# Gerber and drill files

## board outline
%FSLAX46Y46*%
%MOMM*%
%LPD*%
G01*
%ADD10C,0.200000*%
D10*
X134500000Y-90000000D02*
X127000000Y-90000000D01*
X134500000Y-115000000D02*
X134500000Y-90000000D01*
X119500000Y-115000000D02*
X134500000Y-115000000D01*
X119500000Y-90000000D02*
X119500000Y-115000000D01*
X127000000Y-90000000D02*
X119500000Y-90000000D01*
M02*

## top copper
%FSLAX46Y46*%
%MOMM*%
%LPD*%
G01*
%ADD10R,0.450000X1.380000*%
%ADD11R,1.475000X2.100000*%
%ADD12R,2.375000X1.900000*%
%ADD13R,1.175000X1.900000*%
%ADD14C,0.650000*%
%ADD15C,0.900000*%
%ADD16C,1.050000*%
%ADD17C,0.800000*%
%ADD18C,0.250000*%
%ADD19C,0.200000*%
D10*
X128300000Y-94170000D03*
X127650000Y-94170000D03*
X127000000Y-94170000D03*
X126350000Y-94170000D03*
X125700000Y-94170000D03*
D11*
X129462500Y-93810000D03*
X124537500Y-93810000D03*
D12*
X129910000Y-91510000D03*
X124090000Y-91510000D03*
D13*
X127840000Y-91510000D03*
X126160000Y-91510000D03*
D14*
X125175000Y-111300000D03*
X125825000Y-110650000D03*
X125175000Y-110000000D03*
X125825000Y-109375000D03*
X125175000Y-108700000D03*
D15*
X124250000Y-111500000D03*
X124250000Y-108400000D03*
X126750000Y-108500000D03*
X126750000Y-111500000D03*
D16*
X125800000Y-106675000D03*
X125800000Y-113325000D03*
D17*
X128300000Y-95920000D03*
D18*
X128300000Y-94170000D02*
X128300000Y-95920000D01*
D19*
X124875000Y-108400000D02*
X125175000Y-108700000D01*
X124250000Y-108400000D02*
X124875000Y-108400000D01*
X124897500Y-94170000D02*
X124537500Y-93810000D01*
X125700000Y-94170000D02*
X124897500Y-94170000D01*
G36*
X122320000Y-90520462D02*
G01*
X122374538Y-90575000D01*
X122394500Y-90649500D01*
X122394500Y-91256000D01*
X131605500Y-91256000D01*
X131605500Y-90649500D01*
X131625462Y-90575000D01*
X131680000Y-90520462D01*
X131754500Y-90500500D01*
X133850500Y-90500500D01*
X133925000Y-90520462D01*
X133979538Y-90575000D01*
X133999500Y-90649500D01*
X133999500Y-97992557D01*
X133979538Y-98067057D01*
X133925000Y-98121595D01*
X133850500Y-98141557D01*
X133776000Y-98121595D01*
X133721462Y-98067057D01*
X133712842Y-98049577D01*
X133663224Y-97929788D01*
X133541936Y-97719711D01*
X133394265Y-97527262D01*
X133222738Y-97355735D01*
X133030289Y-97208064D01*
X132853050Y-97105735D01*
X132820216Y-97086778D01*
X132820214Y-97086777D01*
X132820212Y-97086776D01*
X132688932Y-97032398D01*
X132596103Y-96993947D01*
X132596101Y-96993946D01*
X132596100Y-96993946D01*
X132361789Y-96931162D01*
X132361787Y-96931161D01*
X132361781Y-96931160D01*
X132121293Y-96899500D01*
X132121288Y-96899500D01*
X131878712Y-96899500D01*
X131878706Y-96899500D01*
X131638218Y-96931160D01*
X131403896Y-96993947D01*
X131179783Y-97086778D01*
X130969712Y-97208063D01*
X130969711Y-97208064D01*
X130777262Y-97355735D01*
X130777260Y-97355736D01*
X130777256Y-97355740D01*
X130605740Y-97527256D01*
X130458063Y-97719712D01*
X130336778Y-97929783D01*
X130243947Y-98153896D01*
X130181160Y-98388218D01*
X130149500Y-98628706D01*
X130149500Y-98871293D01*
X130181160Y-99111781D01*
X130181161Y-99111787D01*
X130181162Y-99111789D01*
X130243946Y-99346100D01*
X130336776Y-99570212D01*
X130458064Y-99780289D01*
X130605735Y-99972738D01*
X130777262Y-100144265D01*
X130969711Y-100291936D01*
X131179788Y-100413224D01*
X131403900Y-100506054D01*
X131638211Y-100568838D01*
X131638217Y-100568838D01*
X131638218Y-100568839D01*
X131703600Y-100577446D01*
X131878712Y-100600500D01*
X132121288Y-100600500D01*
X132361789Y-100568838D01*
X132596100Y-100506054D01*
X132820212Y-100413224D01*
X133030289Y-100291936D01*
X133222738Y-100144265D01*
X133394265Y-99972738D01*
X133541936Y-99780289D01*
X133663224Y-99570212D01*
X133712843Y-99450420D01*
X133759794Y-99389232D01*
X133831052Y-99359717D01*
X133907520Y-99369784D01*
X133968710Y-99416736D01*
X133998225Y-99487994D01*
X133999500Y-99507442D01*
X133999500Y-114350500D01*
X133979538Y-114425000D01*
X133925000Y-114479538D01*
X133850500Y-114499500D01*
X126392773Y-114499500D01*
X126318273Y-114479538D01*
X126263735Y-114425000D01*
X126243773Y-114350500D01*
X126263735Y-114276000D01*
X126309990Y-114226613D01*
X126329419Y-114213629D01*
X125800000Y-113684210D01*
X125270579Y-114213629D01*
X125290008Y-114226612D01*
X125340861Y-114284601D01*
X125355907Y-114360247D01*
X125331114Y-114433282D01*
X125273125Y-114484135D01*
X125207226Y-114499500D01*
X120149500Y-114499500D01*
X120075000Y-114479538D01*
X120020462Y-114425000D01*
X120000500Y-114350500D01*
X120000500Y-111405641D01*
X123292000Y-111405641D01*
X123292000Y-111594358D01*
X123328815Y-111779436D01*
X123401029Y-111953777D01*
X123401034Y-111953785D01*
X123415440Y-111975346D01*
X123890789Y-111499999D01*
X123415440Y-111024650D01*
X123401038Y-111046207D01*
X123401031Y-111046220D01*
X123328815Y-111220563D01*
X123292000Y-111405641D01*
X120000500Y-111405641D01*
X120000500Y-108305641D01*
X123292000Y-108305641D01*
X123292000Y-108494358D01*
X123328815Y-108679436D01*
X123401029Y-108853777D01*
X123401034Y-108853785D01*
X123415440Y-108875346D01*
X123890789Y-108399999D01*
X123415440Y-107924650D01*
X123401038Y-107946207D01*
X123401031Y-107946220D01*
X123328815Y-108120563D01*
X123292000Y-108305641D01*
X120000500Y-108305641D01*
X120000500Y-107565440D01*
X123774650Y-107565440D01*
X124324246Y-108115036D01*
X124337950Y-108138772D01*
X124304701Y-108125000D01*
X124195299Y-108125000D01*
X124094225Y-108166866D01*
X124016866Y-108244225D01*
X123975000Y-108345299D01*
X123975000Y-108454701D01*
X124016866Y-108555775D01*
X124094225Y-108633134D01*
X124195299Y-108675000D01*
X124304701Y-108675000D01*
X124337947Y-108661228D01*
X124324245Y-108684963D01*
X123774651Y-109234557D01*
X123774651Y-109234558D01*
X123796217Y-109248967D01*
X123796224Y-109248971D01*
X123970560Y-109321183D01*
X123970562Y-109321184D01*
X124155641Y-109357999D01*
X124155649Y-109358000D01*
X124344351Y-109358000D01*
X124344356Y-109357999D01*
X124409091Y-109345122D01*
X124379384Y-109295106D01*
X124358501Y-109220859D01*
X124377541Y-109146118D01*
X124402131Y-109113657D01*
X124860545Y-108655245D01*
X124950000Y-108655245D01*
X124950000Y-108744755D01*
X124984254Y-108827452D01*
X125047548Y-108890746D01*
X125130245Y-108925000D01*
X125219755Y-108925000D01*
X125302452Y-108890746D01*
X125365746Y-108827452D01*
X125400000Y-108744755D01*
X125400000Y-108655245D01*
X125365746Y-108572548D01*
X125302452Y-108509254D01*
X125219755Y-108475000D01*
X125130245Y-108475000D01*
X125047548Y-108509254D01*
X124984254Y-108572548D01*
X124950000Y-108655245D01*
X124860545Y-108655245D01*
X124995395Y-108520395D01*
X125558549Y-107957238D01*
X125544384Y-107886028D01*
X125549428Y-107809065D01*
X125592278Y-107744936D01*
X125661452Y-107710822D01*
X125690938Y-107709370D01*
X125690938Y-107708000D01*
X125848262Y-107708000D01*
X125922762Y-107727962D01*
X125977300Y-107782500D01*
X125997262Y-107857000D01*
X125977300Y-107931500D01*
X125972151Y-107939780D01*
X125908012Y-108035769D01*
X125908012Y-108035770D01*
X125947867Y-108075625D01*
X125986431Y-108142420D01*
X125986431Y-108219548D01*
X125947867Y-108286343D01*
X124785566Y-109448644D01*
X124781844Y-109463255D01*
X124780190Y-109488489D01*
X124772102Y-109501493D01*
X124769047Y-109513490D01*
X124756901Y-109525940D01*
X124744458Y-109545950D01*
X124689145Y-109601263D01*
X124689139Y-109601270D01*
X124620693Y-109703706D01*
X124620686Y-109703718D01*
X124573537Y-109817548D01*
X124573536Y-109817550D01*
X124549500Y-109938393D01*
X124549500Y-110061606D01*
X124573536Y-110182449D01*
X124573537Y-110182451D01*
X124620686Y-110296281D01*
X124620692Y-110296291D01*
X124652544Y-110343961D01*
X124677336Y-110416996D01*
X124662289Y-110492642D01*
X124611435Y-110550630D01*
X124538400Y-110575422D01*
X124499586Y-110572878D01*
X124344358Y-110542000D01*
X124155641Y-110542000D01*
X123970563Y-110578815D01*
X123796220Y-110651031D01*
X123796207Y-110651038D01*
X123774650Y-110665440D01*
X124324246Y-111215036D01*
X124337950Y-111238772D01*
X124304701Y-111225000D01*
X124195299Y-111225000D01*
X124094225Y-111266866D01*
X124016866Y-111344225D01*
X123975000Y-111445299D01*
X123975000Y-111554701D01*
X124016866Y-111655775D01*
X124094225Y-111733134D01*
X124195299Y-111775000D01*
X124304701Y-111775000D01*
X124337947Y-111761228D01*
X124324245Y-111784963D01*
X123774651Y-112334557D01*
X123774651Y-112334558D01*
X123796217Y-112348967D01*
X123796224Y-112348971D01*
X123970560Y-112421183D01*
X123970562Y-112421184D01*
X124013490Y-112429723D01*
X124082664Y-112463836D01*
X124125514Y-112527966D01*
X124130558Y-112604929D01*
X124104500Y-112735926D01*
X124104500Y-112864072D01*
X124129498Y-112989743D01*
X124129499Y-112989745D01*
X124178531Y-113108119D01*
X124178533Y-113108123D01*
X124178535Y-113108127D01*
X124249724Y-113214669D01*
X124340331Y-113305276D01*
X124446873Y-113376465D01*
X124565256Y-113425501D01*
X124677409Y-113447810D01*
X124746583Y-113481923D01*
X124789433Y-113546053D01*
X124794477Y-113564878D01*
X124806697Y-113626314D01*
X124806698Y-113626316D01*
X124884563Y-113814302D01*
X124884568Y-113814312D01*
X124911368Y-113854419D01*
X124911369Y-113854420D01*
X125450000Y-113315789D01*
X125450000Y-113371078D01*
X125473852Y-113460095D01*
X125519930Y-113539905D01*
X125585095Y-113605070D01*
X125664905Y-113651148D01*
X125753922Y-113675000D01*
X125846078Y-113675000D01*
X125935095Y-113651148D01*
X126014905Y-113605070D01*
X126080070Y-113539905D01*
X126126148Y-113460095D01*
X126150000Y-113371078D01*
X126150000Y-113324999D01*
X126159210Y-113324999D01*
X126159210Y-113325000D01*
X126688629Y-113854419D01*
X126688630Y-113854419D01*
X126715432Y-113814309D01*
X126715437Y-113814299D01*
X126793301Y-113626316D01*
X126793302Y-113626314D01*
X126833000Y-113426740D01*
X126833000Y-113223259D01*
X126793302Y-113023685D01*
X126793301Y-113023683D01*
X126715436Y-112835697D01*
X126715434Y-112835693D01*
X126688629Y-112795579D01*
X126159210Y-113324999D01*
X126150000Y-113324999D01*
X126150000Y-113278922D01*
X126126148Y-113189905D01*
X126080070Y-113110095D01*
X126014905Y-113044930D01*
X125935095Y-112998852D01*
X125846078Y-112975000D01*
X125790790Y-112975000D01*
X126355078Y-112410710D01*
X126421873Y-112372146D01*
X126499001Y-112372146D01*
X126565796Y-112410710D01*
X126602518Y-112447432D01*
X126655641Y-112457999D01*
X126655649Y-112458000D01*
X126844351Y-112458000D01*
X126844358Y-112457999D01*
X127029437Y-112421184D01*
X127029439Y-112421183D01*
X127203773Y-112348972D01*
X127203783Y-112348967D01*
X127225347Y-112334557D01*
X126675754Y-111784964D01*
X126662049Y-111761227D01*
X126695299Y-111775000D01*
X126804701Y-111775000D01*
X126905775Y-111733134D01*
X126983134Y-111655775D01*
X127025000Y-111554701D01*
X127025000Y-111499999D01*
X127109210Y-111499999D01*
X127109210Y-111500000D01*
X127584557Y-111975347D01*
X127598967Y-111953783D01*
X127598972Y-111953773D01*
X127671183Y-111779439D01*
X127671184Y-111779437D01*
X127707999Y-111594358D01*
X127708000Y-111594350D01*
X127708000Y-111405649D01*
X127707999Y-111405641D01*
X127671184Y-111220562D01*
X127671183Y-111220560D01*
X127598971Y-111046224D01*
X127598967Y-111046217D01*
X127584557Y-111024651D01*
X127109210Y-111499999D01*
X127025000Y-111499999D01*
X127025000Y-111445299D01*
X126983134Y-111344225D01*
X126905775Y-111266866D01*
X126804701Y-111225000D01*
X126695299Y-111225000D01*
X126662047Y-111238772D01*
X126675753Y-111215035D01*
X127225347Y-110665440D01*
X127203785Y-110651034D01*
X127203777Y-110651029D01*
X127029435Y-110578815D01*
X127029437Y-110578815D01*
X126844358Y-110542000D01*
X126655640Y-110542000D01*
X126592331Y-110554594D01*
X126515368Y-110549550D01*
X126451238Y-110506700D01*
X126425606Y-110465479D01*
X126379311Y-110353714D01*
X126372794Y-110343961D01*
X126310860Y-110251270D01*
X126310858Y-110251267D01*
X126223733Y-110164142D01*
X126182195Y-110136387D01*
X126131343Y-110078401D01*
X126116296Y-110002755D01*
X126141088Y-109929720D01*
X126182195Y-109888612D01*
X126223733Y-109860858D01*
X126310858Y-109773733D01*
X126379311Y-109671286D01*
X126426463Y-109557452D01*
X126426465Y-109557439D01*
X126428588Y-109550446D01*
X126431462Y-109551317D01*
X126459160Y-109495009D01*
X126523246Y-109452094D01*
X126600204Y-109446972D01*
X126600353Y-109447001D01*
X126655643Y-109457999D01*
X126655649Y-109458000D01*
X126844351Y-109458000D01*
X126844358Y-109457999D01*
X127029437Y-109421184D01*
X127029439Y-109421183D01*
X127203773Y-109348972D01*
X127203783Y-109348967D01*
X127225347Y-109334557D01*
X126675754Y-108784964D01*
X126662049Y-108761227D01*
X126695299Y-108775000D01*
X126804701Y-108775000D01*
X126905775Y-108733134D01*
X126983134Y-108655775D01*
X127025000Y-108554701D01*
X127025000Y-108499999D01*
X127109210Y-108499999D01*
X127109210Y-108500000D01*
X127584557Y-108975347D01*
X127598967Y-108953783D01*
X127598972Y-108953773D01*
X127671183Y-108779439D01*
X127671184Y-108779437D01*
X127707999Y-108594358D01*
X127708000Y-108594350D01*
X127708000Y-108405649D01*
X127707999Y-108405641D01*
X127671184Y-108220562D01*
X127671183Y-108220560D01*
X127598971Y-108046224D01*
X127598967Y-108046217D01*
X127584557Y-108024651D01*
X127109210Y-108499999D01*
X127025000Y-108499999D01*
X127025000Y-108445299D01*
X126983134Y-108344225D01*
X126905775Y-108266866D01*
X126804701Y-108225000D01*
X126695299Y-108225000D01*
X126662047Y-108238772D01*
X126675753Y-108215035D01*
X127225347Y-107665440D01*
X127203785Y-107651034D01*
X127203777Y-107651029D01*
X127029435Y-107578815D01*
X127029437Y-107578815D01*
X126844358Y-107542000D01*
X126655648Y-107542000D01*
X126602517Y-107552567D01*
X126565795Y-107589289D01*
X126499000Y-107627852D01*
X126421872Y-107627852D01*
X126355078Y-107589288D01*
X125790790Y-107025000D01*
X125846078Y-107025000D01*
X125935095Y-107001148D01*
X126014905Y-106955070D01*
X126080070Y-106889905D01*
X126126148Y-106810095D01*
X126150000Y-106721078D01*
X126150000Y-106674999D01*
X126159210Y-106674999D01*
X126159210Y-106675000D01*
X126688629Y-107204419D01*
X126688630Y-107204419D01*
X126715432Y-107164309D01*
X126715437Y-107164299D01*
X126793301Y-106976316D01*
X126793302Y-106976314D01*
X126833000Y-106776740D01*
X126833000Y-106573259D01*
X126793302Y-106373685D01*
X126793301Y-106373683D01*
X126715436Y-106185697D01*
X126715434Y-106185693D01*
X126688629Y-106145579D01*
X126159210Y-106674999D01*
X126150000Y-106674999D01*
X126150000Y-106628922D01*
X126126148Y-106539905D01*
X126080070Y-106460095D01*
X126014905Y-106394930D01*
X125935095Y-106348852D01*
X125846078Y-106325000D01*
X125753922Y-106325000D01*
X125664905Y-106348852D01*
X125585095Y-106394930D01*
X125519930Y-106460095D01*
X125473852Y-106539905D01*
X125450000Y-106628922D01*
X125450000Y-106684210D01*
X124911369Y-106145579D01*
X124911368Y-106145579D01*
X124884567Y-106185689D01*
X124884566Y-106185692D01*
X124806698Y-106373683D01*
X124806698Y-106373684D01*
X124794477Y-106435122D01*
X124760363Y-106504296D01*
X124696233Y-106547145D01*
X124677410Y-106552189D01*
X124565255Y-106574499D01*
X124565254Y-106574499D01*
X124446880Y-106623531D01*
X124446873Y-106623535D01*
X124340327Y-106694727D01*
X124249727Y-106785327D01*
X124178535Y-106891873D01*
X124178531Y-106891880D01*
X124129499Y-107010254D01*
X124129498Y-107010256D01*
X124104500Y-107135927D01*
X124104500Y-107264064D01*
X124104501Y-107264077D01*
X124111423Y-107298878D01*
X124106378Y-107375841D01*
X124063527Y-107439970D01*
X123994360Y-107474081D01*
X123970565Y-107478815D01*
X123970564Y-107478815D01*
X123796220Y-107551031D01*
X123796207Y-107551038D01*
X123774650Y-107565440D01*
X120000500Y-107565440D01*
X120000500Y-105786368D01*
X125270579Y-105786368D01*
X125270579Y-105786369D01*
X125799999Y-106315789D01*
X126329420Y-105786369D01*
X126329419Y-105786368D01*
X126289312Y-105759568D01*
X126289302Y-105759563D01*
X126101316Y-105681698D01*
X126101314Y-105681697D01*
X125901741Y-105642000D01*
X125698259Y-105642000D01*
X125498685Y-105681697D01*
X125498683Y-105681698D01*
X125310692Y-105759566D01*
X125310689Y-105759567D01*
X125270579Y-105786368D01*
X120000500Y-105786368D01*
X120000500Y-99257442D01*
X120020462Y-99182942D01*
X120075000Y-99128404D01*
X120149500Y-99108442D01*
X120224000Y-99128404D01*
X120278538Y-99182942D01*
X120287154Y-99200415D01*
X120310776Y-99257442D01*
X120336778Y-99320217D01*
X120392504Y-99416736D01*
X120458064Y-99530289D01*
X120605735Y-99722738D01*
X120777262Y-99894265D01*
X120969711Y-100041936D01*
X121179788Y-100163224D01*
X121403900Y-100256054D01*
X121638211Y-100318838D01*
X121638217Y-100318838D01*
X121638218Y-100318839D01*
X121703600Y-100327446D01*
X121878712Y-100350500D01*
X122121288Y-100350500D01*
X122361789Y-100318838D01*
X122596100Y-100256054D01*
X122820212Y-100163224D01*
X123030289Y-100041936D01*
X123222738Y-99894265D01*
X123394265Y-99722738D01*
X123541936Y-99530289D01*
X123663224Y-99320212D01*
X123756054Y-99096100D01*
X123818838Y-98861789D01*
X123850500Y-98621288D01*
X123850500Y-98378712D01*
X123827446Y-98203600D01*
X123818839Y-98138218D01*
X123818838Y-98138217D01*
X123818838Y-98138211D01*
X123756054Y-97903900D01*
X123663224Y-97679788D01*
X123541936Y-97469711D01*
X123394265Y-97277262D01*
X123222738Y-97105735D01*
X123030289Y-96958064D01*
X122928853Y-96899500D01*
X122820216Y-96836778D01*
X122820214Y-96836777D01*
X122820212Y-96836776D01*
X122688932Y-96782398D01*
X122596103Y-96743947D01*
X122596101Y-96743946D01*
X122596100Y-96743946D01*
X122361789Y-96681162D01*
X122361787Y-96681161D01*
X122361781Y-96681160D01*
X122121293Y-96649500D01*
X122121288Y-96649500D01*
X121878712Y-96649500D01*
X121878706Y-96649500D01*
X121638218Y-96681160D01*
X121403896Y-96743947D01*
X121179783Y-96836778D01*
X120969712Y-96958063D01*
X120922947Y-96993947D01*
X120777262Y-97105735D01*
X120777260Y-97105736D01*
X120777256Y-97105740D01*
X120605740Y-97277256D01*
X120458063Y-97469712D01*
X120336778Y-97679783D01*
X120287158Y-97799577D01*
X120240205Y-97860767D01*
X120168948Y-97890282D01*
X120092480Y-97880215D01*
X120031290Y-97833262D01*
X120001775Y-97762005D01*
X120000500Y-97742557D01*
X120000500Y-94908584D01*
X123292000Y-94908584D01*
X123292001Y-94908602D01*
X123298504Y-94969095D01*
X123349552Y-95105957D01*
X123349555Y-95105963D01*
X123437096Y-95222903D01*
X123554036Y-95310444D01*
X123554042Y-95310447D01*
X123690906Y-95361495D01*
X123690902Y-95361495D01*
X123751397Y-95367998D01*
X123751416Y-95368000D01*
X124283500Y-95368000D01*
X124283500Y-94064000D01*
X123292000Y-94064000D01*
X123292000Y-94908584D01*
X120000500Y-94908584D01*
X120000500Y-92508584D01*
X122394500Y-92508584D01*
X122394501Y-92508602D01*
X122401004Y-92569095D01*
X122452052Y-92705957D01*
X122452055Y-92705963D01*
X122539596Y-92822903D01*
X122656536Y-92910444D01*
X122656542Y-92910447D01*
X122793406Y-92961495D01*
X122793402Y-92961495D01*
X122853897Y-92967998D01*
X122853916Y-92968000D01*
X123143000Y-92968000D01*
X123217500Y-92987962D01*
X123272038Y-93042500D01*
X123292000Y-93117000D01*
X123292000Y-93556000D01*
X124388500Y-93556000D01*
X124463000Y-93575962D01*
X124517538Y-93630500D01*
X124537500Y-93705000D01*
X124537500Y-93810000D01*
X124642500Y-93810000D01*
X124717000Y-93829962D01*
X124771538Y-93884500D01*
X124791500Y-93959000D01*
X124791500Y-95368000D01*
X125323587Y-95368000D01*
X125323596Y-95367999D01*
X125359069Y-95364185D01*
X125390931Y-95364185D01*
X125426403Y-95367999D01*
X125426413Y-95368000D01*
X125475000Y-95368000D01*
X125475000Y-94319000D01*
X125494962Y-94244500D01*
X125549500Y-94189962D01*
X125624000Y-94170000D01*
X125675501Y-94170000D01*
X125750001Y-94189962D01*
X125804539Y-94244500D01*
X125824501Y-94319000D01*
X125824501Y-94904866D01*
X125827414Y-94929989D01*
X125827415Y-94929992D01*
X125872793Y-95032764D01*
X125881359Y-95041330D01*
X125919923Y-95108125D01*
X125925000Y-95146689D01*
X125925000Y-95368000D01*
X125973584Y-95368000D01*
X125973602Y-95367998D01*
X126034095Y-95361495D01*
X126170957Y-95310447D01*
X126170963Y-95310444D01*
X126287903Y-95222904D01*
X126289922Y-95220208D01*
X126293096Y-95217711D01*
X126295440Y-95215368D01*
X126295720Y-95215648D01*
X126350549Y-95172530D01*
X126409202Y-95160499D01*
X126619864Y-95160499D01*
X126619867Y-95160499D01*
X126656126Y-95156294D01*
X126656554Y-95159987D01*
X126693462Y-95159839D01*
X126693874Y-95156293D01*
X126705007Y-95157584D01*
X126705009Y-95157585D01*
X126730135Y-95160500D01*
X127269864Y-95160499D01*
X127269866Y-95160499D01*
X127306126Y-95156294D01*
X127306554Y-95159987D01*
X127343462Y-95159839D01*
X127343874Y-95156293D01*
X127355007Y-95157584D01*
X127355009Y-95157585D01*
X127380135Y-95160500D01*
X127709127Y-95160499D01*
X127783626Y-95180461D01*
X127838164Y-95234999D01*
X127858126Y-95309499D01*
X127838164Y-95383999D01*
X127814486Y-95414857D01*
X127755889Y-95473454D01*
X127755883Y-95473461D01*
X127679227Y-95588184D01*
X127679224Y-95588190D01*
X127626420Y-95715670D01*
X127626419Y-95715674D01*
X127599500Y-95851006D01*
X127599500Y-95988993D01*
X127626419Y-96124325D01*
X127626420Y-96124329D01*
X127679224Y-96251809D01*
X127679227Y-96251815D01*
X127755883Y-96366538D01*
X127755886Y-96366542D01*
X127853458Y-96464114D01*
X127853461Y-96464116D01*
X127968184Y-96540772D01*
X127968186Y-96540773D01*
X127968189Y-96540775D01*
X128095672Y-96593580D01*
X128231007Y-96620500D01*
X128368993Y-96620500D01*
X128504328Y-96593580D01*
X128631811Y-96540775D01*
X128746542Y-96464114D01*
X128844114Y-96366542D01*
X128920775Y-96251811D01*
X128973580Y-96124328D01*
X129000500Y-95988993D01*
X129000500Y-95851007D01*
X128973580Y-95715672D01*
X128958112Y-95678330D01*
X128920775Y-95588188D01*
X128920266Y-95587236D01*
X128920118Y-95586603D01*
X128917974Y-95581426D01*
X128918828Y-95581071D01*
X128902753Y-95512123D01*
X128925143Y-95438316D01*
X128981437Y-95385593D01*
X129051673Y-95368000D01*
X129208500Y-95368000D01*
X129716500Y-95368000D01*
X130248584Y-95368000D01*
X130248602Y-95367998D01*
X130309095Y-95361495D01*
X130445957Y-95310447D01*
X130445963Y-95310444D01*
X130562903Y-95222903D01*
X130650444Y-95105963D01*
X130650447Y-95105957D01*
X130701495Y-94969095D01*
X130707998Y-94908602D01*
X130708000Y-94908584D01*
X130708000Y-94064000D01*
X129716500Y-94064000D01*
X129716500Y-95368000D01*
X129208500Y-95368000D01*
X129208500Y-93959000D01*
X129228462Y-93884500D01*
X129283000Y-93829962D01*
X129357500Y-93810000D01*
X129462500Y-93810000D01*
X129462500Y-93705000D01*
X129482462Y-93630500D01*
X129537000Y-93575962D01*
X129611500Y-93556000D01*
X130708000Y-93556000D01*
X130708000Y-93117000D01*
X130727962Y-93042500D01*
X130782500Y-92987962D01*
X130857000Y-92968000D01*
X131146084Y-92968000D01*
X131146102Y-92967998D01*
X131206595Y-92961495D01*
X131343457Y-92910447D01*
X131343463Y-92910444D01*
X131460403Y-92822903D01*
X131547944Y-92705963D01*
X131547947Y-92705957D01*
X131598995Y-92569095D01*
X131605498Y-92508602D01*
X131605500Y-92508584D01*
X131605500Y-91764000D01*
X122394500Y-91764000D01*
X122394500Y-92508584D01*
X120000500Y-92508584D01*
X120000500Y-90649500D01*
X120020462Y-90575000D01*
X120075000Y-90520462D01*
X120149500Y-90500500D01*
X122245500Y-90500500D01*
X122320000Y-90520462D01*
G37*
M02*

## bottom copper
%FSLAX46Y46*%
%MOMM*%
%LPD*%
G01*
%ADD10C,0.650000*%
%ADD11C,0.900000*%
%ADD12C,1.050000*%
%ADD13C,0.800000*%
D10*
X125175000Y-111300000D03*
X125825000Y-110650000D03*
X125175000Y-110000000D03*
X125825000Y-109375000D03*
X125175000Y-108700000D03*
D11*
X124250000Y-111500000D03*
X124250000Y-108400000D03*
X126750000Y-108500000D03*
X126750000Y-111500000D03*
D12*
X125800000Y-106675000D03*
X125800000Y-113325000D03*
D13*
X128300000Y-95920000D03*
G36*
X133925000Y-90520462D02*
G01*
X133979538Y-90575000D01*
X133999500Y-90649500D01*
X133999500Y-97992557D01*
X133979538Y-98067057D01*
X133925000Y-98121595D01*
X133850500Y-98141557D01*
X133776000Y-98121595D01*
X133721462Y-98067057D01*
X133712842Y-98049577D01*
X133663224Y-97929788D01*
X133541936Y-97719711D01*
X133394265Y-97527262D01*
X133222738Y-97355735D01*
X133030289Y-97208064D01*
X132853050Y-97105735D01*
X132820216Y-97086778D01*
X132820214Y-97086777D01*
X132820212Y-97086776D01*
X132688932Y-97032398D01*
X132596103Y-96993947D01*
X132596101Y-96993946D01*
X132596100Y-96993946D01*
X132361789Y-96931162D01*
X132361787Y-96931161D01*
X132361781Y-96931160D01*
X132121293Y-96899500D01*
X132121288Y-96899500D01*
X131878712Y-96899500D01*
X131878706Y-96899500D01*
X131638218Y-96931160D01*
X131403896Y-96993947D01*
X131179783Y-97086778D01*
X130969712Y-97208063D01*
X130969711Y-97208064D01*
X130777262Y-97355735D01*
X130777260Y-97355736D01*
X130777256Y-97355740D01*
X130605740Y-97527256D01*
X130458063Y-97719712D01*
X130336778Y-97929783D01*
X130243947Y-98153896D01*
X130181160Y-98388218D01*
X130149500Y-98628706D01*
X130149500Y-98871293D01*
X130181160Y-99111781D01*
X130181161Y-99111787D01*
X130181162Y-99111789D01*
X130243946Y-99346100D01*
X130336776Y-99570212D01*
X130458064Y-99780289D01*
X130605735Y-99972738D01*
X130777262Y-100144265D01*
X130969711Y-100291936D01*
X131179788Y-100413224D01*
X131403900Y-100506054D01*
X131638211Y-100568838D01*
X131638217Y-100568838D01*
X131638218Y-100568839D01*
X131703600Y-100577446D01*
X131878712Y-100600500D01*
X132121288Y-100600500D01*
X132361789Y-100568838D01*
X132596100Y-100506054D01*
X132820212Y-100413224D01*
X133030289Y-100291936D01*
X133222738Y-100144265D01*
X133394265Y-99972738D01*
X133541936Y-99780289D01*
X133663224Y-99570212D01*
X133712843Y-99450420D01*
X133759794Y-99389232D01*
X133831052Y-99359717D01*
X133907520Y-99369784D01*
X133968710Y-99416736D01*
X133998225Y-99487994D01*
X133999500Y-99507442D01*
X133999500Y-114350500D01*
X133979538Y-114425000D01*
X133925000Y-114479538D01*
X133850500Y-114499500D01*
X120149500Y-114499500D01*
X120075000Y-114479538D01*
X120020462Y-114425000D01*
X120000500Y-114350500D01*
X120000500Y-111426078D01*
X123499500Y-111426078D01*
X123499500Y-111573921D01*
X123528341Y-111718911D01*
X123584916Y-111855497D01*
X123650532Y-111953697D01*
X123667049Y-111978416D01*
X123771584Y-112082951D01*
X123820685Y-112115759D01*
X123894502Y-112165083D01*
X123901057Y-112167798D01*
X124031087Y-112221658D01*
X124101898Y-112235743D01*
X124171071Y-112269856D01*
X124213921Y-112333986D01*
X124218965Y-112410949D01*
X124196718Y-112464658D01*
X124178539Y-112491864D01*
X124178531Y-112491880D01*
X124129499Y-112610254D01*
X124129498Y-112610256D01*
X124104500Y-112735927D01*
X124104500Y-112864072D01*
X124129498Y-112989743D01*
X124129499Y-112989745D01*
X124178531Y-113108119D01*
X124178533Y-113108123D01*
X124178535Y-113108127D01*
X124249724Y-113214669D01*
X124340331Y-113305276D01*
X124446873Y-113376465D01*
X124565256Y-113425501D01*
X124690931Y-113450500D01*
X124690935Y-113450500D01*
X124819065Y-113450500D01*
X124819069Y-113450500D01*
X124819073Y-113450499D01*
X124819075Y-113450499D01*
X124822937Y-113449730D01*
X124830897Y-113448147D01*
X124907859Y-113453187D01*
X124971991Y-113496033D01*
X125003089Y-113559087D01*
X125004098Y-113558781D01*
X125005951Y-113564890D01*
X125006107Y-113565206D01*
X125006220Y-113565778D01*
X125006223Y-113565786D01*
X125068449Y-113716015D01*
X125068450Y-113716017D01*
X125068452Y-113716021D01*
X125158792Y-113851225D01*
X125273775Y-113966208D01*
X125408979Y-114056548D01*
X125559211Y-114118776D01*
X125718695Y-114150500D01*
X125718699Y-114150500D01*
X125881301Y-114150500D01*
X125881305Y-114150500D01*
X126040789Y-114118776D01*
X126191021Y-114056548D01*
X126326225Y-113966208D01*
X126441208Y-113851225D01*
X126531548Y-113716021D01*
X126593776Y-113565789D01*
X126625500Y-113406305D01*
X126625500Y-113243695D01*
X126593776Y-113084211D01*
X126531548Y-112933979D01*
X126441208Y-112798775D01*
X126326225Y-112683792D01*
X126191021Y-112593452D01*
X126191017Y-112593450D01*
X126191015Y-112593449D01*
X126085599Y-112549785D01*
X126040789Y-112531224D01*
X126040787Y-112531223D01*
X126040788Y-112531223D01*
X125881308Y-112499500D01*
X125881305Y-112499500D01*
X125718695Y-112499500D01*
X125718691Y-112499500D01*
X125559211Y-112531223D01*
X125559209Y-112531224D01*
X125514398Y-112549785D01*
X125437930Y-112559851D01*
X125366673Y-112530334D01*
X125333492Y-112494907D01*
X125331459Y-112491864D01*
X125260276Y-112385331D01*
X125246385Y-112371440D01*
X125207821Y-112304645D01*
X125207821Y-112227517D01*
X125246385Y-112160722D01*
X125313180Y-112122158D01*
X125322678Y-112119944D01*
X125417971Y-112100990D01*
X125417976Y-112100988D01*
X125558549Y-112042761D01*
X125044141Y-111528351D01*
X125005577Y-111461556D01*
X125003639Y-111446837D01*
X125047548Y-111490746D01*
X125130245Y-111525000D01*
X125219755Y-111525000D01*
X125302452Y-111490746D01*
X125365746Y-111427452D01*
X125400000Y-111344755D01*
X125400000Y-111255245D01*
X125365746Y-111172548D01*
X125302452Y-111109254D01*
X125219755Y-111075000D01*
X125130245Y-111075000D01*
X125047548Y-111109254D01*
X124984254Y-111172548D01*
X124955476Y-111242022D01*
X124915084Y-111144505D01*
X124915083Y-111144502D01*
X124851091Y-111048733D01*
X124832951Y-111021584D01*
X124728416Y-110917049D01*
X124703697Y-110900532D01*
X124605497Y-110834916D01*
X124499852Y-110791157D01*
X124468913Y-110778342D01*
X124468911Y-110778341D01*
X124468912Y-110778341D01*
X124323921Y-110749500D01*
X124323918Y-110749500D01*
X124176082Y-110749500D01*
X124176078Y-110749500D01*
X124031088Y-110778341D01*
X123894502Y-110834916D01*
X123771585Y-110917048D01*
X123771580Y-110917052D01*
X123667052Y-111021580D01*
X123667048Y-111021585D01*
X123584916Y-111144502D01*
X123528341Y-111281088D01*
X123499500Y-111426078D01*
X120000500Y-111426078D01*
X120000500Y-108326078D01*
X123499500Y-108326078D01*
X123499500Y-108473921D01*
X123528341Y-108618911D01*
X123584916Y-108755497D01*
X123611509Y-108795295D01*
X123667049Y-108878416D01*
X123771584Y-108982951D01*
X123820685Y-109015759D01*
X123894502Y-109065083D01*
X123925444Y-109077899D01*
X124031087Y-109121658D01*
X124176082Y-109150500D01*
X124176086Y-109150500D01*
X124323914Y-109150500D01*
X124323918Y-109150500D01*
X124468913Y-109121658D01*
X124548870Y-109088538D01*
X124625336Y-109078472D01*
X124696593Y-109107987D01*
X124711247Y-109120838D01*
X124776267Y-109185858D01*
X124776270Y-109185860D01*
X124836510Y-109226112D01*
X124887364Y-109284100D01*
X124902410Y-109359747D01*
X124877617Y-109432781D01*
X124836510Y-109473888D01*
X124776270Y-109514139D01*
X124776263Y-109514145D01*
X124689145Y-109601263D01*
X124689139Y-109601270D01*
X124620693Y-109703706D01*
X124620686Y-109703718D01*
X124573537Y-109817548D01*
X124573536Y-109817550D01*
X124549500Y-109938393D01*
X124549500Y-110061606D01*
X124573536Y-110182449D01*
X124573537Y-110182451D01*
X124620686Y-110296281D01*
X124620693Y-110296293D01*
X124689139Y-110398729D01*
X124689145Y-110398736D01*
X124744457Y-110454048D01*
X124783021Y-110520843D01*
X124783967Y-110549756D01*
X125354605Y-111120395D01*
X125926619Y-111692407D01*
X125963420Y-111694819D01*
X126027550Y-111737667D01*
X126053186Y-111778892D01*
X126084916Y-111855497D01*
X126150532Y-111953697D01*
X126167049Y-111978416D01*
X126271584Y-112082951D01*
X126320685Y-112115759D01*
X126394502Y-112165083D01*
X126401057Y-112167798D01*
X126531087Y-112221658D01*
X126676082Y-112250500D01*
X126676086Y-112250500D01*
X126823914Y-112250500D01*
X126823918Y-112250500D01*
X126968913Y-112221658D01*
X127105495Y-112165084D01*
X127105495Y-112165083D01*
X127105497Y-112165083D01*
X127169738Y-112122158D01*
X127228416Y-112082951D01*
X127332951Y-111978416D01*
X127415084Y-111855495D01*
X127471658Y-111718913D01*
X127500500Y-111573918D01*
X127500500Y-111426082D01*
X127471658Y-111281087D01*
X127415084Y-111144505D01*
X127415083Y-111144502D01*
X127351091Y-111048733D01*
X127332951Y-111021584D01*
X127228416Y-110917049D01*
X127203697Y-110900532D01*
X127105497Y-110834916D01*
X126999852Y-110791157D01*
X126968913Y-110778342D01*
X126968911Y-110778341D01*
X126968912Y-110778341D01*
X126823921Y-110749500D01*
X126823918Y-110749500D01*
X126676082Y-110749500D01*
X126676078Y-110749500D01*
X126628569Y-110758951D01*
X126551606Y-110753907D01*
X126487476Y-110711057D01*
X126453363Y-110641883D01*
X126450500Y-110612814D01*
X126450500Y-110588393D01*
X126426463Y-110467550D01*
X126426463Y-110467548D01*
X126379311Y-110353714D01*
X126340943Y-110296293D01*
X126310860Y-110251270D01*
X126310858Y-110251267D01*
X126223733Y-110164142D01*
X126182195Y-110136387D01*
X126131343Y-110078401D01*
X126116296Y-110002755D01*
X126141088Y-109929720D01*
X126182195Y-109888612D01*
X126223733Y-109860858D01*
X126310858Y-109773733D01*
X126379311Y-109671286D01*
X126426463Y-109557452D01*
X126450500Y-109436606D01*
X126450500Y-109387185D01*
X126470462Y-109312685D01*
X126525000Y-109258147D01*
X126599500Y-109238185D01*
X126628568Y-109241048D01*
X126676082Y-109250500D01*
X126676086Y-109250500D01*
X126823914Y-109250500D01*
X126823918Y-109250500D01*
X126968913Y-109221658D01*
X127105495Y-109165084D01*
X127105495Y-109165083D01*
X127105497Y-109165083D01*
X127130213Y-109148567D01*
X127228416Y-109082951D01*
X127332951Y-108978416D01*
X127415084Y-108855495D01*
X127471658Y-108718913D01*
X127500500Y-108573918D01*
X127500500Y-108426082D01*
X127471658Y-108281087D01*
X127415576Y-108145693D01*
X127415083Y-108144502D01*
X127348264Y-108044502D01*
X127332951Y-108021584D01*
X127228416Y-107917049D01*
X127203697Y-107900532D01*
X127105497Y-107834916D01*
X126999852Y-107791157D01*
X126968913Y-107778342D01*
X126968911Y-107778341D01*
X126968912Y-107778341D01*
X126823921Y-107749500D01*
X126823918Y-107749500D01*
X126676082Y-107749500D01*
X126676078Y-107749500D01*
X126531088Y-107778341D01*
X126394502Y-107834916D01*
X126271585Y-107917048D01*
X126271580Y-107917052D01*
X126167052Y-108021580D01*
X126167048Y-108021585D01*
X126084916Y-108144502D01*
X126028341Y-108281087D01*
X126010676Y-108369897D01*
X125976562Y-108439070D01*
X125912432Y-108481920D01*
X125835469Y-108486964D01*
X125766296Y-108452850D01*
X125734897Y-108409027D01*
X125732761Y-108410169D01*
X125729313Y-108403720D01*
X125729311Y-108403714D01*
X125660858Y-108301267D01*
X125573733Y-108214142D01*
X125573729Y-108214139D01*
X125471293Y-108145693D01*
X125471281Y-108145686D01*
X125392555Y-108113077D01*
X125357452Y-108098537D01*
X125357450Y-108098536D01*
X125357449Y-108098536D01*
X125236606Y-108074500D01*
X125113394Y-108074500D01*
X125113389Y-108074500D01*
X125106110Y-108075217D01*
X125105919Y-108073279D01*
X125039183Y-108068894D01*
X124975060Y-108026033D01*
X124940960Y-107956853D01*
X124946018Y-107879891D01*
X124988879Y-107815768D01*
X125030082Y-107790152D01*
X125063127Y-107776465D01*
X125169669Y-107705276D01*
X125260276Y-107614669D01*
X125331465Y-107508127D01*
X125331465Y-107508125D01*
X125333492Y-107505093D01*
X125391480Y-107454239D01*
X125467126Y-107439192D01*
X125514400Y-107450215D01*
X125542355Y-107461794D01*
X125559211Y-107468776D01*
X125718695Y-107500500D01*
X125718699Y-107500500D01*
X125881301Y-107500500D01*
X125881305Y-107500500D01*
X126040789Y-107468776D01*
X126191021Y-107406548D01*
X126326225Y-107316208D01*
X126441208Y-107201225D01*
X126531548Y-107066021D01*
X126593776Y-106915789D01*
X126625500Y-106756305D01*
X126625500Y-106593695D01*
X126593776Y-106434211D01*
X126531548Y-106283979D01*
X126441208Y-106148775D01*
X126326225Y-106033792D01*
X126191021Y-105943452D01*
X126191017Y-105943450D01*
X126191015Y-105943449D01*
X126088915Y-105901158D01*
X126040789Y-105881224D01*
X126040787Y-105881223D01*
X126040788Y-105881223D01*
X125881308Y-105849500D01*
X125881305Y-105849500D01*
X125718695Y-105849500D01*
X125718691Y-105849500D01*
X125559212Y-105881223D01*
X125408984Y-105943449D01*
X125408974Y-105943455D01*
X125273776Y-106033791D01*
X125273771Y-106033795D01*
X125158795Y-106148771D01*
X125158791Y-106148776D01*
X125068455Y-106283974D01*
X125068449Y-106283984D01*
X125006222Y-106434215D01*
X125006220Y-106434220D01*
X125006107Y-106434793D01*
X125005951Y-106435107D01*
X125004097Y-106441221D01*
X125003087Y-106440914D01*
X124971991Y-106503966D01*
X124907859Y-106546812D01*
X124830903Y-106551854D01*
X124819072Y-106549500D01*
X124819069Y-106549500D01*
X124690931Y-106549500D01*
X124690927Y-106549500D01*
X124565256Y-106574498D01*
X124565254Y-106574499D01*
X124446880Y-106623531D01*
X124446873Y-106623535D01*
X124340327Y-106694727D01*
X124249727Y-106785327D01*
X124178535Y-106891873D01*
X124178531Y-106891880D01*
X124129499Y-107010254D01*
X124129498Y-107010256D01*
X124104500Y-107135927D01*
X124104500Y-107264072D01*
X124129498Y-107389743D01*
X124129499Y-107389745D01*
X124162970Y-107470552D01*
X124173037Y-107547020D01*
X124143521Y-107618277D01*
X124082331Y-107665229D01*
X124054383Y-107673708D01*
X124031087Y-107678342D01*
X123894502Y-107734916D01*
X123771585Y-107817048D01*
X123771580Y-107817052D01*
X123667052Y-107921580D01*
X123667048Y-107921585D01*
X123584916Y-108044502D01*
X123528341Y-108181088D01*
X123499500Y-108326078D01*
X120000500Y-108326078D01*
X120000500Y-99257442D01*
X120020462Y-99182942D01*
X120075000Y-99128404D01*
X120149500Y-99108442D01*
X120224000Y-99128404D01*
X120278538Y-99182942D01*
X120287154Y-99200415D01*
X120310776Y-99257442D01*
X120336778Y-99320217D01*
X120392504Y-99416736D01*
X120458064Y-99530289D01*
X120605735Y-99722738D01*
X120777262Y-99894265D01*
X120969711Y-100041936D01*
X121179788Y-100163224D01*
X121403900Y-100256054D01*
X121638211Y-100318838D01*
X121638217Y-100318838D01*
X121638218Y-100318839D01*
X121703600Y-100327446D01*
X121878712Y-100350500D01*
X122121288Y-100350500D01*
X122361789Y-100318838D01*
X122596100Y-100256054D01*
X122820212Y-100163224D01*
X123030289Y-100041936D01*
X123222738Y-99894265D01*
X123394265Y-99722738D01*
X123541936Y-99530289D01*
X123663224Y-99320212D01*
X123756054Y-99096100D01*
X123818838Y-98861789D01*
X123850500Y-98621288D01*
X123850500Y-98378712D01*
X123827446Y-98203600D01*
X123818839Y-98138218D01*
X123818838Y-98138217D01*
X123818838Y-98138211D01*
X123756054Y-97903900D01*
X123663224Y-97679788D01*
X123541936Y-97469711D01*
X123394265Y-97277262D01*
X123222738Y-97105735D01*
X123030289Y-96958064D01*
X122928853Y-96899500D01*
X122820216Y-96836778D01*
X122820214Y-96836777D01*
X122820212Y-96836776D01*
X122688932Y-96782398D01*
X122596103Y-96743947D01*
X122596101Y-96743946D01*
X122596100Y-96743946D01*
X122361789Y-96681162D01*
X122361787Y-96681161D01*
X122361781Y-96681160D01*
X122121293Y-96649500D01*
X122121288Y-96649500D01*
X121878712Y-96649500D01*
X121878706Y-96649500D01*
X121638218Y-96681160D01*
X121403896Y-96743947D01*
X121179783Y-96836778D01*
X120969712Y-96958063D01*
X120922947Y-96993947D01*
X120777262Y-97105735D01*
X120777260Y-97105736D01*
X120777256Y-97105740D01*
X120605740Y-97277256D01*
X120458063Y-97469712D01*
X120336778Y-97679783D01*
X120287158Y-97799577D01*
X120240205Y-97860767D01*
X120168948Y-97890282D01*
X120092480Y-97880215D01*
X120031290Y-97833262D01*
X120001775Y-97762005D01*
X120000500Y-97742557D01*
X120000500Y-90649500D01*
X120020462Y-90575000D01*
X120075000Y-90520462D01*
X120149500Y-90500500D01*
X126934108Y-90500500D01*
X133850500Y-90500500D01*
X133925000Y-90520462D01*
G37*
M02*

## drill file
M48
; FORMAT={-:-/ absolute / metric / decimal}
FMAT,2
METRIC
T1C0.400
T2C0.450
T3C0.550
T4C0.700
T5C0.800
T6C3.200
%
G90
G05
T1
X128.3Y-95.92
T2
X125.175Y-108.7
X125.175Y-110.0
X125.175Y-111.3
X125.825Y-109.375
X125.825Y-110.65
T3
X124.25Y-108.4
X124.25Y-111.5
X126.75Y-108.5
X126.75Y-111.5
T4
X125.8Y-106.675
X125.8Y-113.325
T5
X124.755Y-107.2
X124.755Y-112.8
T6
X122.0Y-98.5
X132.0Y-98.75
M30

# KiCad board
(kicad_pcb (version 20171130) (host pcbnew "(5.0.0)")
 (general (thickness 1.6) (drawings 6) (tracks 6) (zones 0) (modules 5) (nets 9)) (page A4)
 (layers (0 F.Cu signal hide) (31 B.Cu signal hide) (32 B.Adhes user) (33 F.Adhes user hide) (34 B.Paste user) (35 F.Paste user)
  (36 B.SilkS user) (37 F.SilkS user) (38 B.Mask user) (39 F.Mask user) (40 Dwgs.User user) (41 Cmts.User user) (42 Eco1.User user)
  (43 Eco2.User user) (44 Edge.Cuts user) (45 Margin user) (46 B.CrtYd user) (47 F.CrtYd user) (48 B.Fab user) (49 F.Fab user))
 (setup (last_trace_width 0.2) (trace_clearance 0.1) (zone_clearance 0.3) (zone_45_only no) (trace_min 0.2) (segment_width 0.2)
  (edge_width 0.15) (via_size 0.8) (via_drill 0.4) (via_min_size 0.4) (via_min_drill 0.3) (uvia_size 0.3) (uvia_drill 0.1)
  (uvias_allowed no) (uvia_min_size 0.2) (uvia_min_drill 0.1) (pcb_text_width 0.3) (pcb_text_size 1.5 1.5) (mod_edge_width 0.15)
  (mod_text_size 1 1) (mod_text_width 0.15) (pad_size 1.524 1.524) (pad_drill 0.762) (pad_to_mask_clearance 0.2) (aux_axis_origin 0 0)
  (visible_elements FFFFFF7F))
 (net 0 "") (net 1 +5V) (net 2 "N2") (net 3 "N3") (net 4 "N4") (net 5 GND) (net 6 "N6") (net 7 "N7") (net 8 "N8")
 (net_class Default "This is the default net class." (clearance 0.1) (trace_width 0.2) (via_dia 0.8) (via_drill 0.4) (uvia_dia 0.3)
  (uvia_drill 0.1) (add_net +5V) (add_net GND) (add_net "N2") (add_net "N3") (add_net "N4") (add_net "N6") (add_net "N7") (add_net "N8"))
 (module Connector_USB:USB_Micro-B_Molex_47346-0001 (layer F.Cu) (at 127 92.71 180)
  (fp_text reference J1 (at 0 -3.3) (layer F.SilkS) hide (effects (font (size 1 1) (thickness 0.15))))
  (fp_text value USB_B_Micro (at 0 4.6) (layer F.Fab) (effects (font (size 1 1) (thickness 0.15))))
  (pad 1 smd rect (at -1.3 -1.46 180) (size 0.45 1.38) (layers F.Cu F.Paste F.Mask) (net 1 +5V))
  (pad 2 smd rect (at -0.65 -1.46 180) (size 0.45 1.38) (layers F.Cu F.Paste F.Mask) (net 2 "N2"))
  (pad 3 smd rect (at 0 -1.46 180) (size 0.45 1.38) (layers F.Cu F.Paste F.Mask) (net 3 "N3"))
  (pad 4 smd rect (at 0.65 -1.46 180) (size 0.45 1.38) (layers F.Cu F.Paste F.Mask) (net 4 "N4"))
  (pad 5 smd rect (at 1.3 -1.46 180) (size 0.45 1.38) (layers F.Cu F.Paste F.Mask) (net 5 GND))
  (pad 6 smd rect (at -2.4625 -1.1 180) (size 1.475 2.1) (layers F.Cu F.Paste F.Mask) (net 5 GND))
  (pad 6 smd rect (at 2.4625 -1.1 180) (size 1.475 2.1) (layers F.Cu F.Paste F.Mask) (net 5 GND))
  (pad 6 smd rect (at -2.91 1.2 180) (size 2.375 1.9) (layers F.Cu F.Paste F.Mask) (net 5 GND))
  (pad 6 smd rect (at 2.91 1.2 180) (size 2.375 1.9) (layers F.Cu F.Paste F.Mask) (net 5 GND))
  (pad 6 smd rect (at -0.84 1.2 180) (size 1.175 1.9) (layers F.Cu F.Paste F.Mask) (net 5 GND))
  (pad 6 smd rect (at 0.84 1.2 180) (size 1.175 1.9) (layers F.Cu F.Paste F.Mask) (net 5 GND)))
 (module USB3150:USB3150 (layer F.Cu) (at 125.5 110 90)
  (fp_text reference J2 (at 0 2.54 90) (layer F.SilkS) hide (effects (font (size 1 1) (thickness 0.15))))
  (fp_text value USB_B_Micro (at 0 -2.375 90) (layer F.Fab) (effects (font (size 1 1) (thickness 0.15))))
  (pad 1 thru_hole circle (at -1.3 -0.325 90) (size 0.65 0.65) (drill 0.45) (layers *.Cu *.Mask) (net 1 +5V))
  (pad 2 thru_hole circle (at -0.65 0.325 90) (size 0.65 0.65) (drill 0.45) (layers *.Cu *.Mask) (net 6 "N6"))
  (pad 3 thru_hole circle (at 0 -0.325 90) (size 0.65 0.65) (drill 0.45) (layers *.Cu *.Mask) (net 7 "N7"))
  (pad 4 thru_hole circle (at 0.625 0.325 90) (size 0.65 0.65) (drill 0.45) (layers *.Cu *.Mask) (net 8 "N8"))
  (pad 5 thru_hole circle (at 1.3 -0.325 90) (size 0.65 0.65) (drill 0.45) (layers *.Cu *.Mask) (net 5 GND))
  (pad 6 thru_hole circle (at -1.5 -1.25 90) (size 0.9 0.9) (drill 0.55) (layers *.Cu *.Mask) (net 5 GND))
  (pad 6 thru_hole circle (at 1.6 -1.25 90) (size 0.9 0.9) (drill 0.55) (layers *.Cu *.Mask) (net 5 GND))
  (pad 6 thru_hole circle (at 1.5 1.25 90) (size 0.9 0.9) (drill 0.55) (layers *.Cu *.Mask) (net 5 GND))
  (pad 6 thru_hole circle (at -1.5 1.25 90) (size 0.9 0.9) (drill 0.55) (layers *.Cu *.Mask) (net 5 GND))
  (pad 6 thru_hole circle (at 3.325 0.3 90) (size 1.05 1.05) (drill 0.7) (layers *.Cu *.Mask) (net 5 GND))
  (pad 6 thru_hole circle (at -3.325 0.3 90) (size 1.05 1.05) (drill 0.7) (layers *.Cu *.Mask) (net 5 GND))
  (pad "" np_thru_hole circle (at 2.8 -0.745 90) (size 0.8 0.8) (drill 0.8) (layers *.Cu *.Mask))
  (pad "" np_thru_hole circle (at -2.8 -0.745 90) (size 0.8 0.8) (drill 0.8) (layers *.Cu *.Mask)))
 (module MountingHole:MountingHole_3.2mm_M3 (layer F.Cu) (at 122 98.5)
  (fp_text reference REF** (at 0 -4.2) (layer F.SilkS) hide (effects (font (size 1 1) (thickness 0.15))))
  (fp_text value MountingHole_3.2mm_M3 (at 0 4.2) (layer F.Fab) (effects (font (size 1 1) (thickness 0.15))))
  (pad 1 np_thru_hole circle (at 0 0) (size 3.2 3.2) (drill 3.2) (layers *.Cu *.Mask)))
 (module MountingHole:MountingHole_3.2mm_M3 (layer F.Cu) (at 132 98.75)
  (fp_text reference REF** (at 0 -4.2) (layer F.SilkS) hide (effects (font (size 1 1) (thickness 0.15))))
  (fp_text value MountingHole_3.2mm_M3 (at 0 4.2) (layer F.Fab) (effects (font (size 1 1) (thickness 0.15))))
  (pad 1 np_thru_hole circle (at 0 0) (size 3.2 3.2) (drill 3.2) (layers *.Cu *.Mask)))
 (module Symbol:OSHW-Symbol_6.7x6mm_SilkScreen (layer F.Cu) (at 127 102.5)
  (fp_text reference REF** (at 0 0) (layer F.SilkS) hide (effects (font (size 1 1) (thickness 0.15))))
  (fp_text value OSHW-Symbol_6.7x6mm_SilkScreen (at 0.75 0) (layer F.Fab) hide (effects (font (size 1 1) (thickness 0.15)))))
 (gr_line (start 134.5 90) (end 127 90) (layer Edge.Cuts) (width 0.2))
 (gr_line (start 134.5 115) (end 134.5 90) (layer Edge.Cuts) (width 0.2))
 (gr_line (start 119.5 115) (end 134.5 115) (layer Edge.Cuts) (width 0.2))
 (gr_line (start 119.5 90) (end 119.5 115) (layer Edge.Cuts) (width 0.2))
 (gr_line (start 127 90) (end 119.5 90) (layer Edge.Cuts) (width 0.2))
 (via (at 128.3 95.92) (size 0.8) (drill 0.4) (layers F.Cu B.Cu) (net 1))
 (segment (start 128.3 94.17) (end 128.3 95.92) (width 0.25) (layer F.Cu) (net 1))
 (segment (start 124.875 108.4) (end 125.175 108.7) (width 0.2) (layer F.Cu) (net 5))
 (segment (start 124.25 108.4) (end 124.875 108.4) (width 0.2) (layer F.Cu) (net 5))
 (segment (start 124.8975 94.17) (end 124.5375 93.81) (width 0.2) (layer F.Cu) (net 5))
 (segment (start 125.7 94.17) (end 124.8975 94.17) (width 0.2) (layer F.Cu) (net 5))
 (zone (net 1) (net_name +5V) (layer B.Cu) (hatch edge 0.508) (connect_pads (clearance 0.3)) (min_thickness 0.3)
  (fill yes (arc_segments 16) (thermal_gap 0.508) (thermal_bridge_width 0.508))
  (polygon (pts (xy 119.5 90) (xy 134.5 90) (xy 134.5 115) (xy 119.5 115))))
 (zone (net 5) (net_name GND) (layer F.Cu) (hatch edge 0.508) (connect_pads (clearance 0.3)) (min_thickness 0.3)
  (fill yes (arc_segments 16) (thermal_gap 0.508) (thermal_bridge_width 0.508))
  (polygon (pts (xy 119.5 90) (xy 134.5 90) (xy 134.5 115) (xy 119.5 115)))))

